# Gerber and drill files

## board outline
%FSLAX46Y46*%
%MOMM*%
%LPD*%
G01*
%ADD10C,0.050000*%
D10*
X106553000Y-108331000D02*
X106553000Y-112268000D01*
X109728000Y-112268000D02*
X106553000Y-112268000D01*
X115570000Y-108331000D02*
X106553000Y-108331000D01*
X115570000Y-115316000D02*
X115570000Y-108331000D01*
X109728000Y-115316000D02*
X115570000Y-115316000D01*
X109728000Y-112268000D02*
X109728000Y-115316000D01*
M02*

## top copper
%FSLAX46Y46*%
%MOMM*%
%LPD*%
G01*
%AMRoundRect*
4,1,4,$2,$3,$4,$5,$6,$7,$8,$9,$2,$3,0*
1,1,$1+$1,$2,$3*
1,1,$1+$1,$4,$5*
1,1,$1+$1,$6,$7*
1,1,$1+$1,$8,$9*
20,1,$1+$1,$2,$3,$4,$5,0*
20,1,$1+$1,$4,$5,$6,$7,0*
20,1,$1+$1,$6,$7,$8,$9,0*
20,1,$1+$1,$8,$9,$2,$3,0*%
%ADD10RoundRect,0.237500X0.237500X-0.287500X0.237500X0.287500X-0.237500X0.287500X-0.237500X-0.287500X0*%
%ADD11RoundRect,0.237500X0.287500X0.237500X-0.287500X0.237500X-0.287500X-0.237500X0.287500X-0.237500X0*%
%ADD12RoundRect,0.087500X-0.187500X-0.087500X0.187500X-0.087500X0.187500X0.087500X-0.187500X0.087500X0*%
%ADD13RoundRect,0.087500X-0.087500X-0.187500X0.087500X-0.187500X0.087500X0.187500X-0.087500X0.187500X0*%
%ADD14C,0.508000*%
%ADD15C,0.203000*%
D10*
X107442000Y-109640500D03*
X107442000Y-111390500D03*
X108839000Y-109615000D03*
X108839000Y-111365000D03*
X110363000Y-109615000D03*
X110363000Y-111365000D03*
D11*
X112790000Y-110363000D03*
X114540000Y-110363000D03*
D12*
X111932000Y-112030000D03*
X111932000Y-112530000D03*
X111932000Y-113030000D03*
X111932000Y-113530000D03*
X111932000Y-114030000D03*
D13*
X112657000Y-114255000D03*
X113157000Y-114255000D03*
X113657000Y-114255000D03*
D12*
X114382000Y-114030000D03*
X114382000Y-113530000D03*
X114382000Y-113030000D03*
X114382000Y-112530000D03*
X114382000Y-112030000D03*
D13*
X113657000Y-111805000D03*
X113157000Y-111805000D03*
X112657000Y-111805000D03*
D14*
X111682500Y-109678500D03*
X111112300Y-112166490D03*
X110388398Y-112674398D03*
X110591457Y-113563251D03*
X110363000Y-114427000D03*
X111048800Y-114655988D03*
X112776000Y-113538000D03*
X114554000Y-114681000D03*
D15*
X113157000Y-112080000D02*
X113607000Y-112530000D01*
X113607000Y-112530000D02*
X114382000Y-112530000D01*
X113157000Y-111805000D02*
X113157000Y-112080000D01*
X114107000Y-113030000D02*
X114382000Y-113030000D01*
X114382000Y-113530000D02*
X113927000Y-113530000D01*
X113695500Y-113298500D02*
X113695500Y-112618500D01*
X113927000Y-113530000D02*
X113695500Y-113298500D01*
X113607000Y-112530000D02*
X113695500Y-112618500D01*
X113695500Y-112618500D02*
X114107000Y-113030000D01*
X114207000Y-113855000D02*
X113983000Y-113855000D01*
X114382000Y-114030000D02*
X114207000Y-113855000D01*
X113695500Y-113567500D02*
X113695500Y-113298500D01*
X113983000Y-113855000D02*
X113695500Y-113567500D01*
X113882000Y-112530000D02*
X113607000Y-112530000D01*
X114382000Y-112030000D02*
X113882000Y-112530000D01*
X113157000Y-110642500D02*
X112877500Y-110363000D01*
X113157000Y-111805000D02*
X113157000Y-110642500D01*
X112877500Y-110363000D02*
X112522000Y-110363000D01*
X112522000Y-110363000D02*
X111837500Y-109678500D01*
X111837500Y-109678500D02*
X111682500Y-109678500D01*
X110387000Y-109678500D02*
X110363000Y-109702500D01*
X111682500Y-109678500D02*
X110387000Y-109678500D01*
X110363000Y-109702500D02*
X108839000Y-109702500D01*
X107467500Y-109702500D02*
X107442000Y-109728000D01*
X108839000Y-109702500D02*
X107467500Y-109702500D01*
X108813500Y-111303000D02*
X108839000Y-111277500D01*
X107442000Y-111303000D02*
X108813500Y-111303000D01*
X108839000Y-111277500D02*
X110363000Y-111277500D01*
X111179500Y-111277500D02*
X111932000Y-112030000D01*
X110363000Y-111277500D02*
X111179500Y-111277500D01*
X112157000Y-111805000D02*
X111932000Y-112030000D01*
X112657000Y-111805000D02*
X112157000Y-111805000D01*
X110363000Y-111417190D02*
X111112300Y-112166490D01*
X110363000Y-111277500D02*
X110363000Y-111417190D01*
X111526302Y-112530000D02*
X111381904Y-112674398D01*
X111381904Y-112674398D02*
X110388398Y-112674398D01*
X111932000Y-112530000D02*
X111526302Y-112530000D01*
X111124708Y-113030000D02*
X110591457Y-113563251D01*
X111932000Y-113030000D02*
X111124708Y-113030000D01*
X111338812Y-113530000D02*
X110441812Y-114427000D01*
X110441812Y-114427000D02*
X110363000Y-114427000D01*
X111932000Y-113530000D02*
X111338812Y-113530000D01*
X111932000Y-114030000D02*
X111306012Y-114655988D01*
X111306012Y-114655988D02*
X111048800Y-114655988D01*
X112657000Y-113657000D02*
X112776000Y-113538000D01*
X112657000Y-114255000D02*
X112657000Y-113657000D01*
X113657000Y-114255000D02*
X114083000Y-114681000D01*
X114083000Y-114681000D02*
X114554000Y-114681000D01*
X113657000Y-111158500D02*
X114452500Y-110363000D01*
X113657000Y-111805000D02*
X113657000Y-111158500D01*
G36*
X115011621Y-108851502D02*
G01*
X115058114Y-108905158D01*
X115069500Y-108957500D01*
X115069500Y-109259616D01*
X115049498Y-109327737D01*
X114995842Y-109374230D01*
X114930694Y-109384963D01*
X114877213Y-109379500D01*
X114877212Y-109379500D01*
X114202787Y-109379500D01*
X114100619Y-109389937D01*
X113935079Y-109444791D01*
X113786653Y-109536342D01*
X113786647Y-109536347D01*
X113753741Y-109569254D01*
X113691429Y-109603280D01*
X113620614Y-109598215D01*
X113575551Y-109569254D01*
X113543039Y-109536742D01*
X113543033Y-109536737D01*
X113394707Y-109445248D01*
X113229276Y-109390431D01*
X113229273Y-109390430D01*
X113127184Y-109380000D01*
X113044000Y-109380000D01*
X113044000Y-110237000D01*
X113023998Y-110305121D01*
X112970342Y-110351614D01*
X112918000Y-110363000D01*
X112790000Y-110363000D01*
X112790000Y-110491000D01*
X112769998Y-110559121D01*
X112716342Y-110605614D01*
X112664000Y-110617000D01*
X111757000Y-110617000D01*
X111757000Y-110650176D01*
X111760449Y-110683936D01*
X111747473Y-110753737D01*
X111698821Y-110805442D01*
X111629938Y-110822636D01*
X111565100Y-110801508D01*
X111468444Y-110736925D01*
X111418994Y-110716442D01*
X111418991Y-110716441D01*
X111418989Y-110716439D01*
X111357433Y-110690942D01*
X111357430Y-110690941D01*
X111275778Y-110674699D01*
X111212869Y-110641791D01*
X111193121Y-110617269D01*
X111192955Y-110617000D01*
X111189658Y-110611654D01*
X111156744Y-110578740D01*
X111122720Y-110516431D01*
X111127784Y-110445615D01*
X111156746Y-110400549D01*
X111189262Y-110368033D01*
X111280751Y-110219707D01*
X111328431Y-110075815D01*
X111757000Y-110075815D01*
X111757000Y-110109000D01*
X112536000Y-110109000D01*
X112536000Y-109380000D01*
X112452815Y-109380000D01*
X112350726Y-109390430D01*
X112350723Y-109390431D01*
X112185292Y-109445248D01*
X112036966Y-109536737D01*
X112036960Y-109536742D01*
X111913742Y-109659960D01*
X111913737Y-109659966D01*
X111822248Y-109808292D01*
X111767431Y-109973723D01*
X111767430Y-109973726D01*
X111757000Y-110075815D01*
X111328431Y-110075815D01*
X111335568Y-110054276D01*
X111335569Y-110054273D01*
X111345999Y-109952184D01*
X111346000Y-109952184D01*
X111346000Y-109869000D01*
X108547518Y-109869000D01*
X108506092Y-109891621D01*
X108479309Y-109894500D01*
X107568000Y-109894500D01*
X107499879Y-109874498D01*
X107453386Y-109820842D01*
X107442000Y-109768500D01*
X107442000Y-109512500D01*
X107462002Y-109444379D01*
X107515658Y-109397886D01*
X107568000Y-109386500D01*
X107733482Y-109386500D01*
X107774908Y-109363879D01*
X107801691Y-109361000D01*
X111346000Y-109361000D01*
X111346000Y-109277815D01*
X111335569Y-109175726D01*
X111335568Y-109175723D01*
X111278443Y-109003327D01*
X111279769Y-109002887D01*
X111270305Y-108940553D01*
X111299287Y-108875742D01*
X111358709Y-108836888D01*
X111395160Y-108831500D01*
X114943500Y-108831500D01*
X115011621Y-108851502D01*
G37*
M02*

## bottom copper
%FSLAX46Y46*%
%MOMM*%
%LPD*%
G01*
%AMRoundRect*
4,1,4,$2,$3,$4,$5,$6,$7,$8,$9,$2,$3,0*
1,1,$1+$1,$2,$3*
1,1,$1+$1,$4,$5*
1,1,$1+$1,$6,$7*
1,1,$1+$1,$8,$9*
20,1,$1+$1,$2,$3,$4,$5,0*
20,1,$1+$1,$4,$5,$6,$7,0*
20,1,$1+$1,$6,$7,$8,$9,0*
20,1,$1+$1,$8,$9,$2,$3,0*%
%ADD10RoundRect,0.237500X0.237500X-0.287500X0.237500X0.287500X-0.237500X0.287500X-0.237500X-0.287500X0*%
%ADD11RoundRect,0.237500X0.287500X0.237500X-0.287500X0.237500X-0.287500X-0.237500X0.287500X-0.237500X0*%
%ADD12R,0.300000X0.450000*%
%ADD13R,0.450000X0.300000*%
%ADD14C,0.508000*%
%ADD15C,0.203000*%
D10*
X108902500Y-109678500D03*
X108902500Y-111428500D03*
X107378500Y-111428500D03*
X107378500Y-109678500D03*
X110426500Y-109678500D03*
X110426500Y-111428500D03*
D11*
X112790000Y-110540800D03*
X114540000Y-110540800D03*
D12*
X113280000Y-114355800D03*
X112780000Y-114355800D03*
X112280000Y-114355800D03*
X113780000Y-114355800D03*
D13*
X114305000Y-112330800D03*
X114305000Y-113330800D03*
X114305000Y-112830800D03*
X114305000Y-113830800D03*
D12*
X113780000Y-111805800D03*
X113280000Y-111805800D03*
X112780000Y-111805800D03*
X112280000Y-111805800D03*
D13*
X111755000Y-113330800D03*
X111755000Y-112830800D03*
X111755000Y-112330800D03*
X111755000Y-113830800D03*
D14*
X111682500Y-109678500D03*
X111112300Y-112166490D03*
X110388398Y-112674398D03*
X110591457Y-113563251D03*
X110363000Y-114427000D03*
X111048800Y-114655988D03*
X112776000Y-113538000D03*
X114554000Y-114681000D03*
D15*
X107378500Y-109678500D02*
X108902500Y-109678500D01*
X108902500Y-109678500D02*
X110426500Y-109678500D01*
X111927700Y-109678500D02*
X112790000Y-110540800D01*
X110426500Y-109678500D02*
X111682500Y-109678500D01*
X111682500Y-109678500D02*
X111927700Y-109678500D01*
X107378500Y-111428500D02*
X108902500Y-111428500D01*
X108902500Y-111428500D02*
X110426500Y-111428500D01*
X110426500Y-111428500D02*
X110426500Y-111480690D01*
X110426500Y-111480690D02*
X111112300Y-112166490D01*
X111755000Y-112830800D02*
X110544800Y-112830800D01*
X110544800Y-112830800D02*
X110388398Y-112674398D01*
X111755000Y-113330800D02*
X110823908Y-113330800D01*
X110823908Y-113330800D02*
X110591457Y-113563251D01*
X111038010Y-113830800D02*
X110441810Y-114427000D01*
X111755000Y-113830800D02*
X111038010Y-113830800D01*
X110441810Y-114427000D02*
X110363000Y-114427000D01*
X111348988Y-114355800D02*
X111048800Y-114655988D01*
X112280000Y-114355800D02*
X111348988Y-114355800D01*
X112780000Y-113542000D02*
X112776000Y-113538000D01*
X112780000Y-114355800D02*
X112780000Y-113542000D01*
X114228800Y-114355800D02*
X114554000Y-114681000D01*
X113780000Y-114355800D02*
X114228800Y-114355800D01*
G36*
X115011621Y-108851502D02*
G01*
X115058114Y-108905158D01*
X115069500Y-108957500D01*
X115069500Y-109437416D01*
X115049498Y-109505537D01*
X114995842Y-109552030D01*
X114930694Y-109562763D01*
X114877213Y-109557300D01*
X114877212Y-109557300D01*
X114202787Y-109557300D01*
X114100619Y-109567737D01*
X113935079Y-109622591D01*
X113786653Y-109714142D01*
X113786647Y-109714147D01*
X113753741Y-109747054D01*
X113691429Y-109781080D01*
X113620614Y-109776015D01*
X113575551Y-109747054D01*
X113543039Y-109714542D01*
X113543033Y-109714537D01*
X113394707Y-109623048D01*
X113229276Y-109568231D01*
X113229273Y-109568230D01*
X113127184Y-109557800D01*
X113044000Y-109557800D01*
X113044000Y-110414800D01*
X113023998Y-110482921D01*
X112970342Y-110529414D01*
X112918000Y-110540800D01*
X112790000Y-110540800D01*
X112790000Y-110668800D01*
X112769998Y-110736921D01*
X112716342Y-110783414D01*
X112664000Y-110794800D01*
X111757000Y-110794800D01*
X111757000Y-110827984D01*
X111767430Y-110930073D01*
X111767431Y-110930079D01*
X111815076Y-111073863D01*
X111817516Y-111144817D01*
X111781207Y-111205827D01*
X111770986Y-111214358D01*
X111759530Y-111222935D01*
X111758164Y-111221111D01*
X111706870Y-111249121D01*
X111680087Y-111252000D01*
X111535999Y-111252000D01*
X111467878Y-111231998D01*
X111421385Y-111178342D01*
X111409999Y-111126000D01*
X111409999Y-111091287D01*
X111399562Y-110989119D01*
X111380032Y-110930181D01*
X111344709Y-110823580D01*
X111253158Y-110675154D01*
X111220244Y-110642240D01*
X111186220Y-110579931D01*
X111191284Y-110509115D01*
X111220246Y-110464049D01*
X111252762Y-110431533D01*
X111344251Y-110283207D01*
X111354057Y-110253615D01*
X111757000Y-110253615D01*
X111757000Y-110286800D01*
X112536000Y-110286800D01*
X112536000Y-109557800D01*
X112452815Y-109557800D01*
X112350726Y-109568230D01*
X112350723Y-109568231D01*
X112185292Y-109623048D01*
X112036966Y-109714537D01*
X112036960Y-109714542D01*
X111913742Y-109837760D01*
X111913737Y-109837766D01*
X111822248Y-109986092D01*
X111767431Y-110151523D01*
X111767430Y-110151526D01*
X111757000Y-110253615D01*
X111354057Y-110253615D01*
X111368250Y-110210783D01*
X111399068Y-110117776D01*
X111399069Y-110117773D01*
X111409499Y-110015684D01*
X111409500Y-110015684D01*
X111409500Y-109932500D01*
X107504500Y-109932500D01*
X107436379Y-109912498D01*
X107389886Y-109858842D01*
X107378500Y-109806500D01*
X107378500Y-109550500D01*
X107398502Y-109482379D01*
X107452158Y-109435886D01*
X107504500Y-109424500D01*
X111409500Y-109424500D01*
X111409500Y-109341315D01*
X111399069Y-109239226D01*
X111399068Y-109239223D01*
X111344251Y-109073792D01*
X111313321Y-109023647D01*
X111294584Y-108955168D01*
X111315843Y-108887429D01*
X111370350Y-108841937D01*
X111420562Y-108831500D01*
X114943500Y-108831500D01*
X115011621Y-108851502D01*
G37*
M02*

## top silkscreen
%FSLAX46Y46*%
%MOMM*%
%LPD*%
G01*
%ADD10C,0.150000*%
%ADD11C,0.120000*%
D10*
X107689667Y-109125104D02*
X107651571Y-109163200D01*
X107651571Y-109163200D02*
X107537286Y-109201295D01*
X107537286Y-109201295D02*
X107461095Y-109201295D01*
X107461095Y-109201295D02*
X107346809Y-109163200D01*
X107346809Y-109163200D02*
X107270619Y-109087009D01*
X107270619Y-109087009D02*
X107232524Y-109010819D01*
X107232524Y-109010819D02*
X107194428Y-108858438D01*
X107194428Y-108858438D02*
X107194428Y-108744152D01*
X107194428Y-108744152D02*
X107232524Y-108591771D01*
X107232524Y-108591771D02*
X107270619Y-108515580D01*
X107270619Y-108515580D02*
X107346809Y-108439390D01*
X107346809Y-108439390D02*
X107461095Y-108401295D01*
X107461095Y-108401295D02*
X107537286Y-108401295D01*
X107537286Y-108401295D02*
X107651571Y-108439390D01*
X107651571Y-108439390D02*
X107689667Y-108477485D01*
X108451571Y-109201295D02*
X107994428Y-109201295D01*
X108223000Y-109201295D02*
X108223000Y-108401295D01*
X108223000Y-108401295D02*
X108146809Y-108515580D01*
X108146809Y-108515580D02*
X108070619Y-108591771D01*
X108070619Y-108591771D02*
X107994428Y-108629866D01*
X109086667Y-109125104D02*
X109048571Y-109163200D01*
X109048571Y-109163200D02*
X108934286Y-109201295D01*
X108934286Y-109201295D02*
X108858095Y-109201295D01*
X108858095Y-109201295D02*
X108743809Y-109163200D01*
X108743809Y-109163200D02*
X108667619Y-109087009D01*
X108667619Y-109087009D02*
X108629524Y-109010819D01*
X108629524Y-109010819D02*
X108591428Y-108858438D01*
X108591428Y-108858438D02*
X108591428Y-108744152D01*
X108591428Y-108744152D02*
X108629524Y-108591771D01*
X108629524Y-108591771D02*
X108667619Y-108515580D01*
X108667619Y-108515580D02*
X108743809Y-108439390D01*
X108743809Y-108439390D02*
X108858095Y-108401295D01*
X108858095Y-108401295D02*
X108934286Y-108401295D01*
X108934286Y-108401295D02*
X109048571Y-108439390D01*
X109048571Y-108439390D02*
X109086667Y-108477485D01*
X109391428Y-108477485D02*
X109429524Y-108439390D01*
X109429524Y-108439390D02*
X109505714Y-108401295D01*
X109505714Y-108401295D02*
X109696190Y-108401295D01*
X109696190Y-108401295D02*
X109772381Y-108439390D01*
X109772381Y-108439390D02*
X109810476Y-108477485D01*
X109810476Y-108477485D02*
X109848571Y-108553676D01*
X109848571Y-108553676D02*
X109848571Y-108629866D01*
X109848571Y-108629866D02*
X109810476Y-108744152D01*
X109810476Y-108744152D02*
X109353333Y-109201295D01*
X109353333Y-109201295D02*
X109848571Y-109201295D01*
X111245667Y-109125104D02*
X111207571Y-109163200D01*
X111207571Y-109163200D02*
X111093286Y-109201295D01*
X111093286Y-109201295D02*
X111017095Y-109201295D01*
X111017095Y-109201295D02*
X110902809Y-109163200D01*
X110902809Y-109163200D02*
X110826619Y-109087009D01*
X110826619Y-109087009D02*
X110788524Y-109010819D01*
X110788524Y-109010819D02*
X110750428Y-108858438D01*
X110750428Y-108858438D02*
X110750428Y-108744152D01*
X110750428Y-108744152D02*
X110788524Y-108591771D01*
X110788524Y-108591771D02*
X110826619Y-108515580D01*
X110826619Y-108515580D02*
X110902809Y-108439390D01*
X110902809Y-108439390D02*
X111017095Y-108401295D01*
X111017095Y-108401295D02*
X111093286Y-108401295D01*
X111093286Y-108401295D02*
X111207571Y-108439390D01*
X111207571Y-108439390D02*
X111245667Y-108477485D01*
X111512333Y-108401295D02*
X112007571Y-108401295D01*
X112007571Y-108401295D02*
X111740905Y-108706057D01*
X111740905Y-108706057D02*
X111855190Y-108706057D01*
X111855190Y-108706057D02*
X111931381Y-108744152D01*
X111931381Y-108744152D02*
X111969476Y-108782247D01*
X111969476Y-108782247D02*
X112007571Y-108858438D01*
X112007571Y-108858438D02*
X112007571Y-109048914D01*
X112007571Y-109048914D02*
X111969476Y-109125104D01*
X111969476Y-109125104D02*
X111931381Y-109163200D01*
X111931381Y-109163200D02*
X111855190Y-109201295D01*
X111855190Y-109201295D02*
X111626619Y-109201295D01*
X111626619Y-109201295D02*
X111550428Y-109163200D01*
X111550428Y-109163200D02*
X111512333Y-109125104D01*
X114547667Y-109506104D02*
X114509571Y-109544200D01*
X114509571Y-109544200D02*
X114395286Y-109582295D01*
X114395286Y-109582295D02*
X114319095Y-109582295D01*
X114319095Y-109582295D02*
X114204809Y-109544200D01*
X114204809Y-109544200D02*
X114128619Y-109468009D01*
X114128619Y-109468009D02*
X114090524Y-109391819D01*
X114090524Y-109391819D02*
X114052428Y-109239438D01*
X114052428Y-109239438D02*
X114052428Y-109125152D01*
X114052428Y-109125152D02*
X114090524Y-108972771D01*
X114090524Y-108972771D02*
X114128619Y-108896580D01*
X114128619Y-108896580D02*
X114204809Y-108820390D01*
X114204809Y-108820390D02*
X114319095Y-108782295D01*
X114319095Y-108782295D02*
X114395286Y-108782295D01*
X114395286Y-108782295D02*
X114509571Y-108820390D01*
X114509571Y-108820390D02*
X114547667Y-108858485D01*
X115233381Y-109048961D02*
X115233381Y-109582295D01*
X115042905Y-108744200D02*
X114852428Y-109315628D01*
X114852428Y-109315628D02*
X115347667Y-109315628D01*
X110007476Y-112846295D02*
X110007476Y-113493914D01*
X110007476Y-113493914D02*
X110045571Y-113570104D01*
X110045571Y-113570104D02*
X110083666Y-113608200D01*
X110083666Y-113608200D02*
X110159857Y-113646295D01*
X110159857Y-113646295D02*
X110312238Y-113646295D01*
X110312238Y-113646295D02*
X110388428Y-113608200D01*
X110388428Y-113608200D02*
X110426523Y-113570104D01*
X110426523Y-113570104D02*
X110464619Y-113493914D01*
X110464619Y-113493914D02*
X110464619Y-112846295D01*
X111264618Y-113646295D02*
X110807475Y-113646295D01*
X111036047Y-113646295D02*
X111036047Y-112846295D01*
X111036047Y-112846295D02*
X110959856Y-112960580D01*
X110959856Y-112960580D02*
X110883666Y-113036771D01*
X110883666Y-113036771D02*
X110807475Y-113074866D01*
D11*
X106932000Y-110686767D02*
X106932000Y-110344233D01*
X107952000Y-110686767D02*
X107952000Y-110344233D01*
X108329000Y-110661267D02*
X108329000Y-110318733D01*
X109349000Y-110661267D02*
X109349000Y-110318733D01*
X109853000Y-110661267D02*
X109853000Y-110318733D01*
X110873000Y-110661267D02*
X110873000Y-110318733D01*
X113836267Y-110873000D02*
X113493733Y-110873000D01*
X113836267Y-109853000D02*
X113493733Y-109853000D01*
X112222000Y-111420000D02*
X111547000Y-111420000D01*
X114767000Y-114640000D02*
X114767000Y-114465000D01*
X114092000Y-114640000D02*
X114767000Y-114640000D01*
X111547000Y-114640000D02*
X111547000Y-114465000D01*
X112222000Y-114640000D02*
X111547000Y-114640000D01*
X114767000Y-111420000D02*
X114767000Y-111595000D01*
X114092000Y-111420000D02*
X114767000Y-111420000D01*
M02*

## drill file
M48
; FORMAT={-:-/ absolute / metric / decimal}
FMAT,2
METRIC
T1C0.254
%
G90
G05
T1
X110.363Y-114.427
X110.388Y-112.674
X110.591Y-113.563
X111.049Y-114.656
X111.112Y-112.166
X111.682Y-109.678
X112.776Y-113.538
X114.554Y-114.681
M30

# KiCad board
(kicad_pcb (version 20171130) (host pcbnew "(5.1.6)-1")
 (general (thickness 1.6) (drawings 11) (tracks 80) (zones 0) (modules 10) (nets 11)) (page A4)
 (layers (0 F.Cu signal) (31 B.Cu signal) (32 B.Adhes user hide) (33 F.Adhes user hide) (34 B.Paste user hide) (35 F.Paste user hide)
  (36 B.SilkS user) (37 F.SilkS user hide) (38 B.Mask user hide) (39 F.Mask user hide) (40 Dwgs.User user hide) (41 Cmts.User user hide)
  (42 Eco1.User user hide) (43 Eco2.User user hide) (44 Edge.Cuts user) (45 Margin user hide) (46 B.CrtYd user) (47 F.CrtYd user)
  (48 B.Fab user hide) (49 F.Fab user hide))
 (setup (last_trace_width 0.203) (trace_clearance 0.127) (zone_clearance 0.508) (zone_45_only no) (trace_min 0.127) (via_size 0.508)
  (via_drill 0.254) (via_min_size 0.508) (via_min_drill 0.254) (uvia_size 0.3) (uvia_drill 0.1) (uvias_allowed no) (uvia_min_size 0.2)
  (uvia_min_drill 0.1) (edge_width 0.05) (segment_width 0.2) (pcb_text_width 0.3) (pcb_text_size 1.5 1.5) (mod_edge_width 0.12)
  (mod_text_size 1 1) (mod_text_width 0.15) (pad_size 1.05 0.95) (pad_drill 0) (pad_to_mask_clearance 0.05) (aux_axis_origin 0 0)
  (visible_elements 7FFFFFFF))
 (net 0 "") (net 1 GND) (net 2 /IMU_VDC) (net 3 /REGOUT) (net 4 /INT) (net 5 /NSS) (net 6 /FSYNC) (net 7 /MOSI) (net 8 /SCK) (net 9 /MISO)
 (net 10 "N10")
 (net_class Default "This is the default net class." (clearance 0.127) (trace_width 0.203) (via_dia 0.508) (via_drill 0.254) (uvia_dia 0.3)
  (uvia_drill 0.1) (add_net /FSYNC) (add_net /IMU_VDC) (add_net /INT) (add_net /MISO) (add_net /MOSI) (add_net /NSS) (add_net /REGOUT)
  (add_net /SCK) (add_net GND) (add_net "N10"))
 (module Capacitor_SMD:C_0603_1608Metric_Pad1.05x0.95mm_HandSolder (layer F.Cu) (at 107.442 110.5155 90)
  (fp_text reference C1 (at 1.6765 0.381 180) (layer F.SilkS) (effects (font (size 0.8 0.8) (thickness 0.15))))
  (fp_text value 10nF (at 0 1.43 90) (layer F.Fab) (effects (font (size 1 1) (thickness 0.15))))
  (fp_line (start -0.171267 -0.51) (end 0.171267 -0.51) (layer F.SilkS) (width 0.12))
  (fp_line (start -0.171267 0.51) (end 0.171267 0.51) (layer F.SilkS) (width 0.12))
  (pad 2 smd roundrect (at 0.875 0 90) (size 1.05 0.95) (layers F.Cu F.Paste F.Mask) (roundrect_rratio 0.25) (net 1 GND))
  (pad 1 smd roundrect (at -0.875 0 90) (size 1.05 0.95) (layers F.Cu F.Paste F.Mask) (roundrect_rratio 0.25) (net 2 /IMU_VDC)))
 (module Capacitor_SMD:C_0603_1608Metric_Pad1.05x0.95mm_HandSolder (layer F.Cu) (at 108.839 110.49 90)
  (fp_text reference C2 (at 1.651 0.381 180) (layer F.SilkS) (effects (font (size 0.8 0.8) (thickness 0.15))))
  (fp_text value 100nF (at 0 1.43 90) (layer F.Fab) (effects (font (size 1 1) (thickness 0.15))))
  (fp_line (start -0.171267 -0.51) (end 0.171267 -0.51) (layer F.SilkS) (width 0.12))
  (fp_line (start -0.171267 0.51) (end 0.171267 0.51) (layer F.SilkS) (width 0.12))
  (pad 2 smd roundrect (at 0.875 0 90) (size 1.05 0.95) (layers F.Cu F.Paste F.Mask) (roundrect_rratio 0.25) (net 1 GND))
  (pad 1 smd roundrect (at -0.875 0 90) (size 1.05 0.95) (layers F.Cu F.Paste F.Mask) (roundrect_rratio 0.25) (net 2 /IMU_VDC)))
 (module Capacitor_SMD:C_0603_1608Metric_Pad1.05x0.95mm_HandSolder (layer F.Cu) (at 110.363 110.49 90)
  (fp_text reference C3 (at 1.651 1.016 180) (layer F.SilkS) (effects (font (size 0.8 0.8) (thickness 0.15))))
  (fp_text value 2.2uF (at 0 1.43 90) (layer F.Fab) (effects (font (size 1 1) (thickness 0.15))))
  (fp_line (start -0.171267 -0.51) (end 0.171267 -0.51) (layer F.SilkS) (width 0.12))
  (fp_line (start -0.171267 0.51) (end 0.171267 0.51) (layer F.SilkS) (width 0.12))
  (pad 2 smd roundrect (at 0.875 0 90) (size 1.05 0.95) (layers F.Cu F.Paste F.Mask) (roundrect_rratio 0.25) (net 1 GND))
  (pad 1 smd roundrect (at -0.875 0 90) (size 1.05 0.95) (layers F.Cu F.Paste F.Mask) (roundrect_rratio 0.25) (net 2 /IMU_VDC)))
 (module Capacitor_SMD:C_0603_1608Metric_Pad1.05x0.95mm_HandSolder (layer F.Cu) (at 113.665 110.363 180)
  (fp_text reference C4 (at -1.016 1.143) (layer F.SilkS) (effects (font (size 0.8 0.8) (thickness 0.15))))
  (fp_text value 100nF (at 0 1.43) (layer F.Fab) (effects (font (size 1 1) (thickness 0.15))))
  (fp_line (start -0.171267 -0.51) (end 0.171267 -0.51) (layer F.SilkS) (width 0.12))
  (fp_line (start -0.171267 0.51) (end 0.171267 0.51) (layer F.SilkS) (width 0.12))
  (pad 2 smd roundrect (at 0.875 0 180) (size 1.05 0.95) (layers F.Cu F.Paste F.Mask) (roundrect_rratio 0.25) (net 1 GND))
  (pad 1 smd roundrect (at -0.875 0 180) (size 1.05 0.95) (layers F.Cu F.Paste F.Mask) (roundrect_rratio 0.25) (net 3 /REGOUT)))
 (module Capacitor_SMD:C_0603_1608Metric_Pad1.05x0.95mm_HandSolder (layer B.Cu) (at 108.9025 110.5535 90)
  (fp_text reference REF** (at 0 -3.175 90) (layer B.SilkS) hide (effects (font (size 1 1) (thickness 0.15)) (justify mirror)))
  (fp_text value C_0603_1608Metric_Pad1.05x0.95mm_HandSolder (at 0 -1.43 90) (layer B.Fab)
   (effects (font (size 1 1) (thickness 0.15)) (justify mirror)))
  (pad 2 smd roundrect (at 0.875 0 90) (size 1.05 0.95) (layers B.Cu B.Paste B.Mask) (roundrect_rratio 0.25) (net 1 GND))
  (pad 1 smd roundrect (at -0.875 0 90) (size 1.05 0.95) (layers B.Cu B.Paste B.Mask) (roundrect_rratio 0.25) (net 2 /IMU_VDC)))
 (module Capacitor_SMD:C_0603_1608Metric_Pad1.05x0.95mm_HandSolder (layer B.Cu) (at 107.3785 110.5535 90)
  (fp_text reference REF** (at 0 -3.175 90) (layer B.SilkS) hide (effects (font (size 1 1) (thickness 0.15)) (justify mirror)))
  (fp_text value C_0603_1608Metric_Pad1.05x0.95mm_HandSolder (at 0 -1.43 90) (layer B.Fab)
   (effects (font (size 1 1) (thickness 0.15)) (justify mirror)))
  (pad 1 smd roundrect (at -0.875 0 90) (size 1.05 0.95) (layers B.Cu B.Paste B.Mask) (roundrect_rratio 0.25) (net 2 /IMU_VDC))
  (pad 2 smd roundrect (at 0.875 0 90) (size 1.05 0.95) (layers B.Cu B.Paste B.Mask) (roundrect_rratio 0.25) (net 1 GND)))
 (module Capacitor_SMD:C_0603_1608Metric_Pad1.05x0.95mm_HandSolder (layer B.Cu) (at 110.4265 110.5535 90)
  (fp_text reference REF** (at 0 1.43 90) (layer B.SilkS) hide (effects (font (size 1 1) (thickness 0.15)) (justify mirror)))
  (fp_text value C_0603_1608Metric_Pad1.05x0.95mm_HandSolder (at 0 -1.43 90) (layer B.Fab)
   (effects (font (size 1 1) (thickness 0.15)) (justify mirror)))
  (pad 2 smd roundrect (at 0.875 0 90) (size 1.05 0.95) (layers B.Cu B.Paste B.Mask) (roundrect_rratio 0.25) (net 1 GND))
  (pad 1 smd roundrect (at -0.875 0 90) (size 1.05 0.95) (layers B.Cu B.Paste B.Mask) (roundrect_rratio 0.25) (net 2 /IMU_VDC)))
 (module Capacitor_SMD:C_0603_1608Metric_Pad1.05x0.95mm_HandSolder (layer B.Cu) (at 113.665 110.5408 180)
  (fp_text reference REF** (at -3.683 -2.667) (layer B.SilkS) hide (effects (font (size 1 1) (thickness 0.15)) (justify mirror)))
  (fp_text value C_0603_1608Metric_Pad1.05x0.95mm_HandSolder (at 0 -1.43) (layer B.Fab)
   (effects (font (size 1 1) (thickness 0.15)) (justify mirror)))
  (pad 2 smd roundrect (at 0.875 0 180) (size 1.05 0.95) (layers B.Cu B.Paste B.Mask) (roundrect_rratio 0.25) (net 1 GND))
  (pad 1 smd roundrect (at -0.875 0 180) (size 1.05 0.95) (layers B.Cu B.Paste B.Mask) (roundrect_rratio 0.25)))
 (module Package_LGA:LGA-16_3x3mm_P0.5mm (layer B.Cu) (at 113.03 113.0808 270)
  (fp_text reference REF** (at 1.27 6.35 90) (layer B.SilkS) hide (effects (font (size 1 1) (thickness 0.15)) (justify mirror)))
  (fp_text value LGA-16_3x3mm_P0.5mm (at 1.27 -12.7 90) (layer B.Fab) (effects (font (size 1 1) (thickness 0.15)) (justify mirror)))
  (pad 10 smd rect (at 1.275 -0.25 180) (size 0.3 0.45) (layers B.Cu B.Paste B.Mask))
  (pad 11 smd rect (at 1.275 0.25 180) (size 0.3 0.45) (layers B.Cu B.Paste B.Mask) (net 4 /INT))
  (pad 12 smd rect (at 1.275 0.75 180) (size 0.3 0.45) (layers B.Cu B.Paste B.Mask) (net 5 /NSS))
  (pad 9 smd rect (at 1.275 -0.75 180) (size 0.3 0.45) (layers B.Cu B.Paste B.Mask) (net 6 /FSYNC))
  (pad 5 smd rect (at -0.75 -1.275 270) (size 0.3 0.45) (layers B.Cu B.Paste B.Mask))
  (pad 7 smd rect (at 0.25 -1.275 270) (size 0.3 0.45) (layers B.Cu B.Paste B.Mask))
  (pad 6 smd rect (at -0.25 -1.275 270) (size 0.3 0.45) (layers B.Cu B.Paste B.Mask))
  (pad 8 smd rect (at 0.75 -1.275 270) (size 0.3 0.45) (layers B.Cu B.Paste B.Mask))
  (pad 4 smd rect (at -1.275 -0.75 180) (size 0.3 0.45) (layers B.Cu B.Paste B.Mask))
  (pad 3 smd rect (at -1.275 -0.25 180) (size 0.3 0.45) (layers B.Cu B.Paste B.Mask))
  (pad 2 smd rect (at -1.275 0.25 180) (size 0.3 0.45) (layers B.Cu B.Paste B.Mask))
  (pad 1 smd rect (at -1.275 0.75 180) (size 0.3 0.45) (layers B.Cu B.Paste B.Mask))
  (pad 14 smd rect (at 0.25 1.275 270) (size 0.3 0.45) (layers B.Cu B.Paste B.Mask) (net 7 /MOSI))
  (pad 15 smd rect (at -0.25 1.275 270) (size 0.3 0.45) (layers B.Cu B.Paste B.Mask) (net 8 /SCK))
  (pad 16 smd rect (at -0.75 1.275 270) (size 0.3 0.45) (layers B.Cu B.Paste B.Mask))
  (pad 13 smd rect (at 0.75 1.275 270) (size 0.3 0.45) (layers B.Cu B.Paste B.Mask) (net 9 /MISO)))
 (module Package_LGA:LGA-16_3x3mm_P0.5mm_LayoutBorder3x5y (layer F.Cu) (at 113.157 113.03)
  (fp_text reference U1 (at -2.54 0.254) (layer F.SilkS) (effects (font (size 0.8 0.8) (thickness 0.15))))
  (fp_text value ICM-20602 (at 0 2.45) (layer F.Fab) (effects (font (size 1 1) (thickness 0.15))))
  (fp_line (start -0.935 -1.61) (end -1.61 -1.61) (layer F.SilkS) (width 0.12))
  (fp_line (start 1.61 1.61) (end 1.61 1.435) (layer F.SilkS) (width 0.12))
  (fp_line (start 0.935 1.61) (end 1.61 1.61) (layer F.SilkS) (width 0.12))
  (fp_line (start -1.61 1.61) (end -1.61 1.435) (layer F.SilkS) (width 0.12))
  (fp_line (start -0.935 1.61) (end -1.61 1.61) (layer F.SilkS) (width 0.12))
  (fp_line (start 1.61 -1.61) (end 1.61 -1.435) (layer F.SilkS) (width 0.12))
  (fp_line (start 0.935 -1.61) (end 1.61 -1.61) (layer F.SilkS) (width 0.12))
  (pad 1 smd roundrect (at -1.225 -1) (size 0.55 0.35) (layers F.Cu F.Paste F.Mask) (roundrect_rratio 0.25) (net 2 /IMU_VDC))
  (pad 2 smd roundrect (at -1.225 -0.5) (size 0.55 0.35) (layers F.Cu F.Paste F.Mask) (roundrect_rratio 0.25) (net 8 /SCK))
  (pad 3 smd roundrect (at -1.225 0) (size 0.55 0.35) (layers F.Cu F.Paste F.Mask) (roundrect_rratio 0.25) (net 7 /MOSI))
  (pad 4 smd roundrect (at -1.225 0.5) (size 0.55 0.35) (layers F.Cu F.Paste F.Mask) (roundrect_rratio 0.25) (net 9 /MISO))
  (pad 5 smd roundrect (at -1.225 1) (size 0.55 0.35) (layers F.Cu F.Paste F.Mask) (roundrect_rratio 0.25) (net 5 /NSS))
  (pad 6 smd roundrect (at -0.5 1.225) (size 0.35 0.55) (layers F.Cu F.Paste F.Mask) (roundrect_rratio 0.25) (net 4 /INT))
  (pad 7 smd roundrect (at 0 1.225) (size 0.35 0.55) (layers F.Cu F.Paste F.Mask) (roundrect_rratio 0.25) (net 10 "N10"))
  (pad 8 smd roundrect (at 0.5 1.225) (size 0.35 0.55) (layers F.Cu F.Paste F.Mask) (roundrect_rratio 0.25) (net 6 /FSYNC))
  (pad 9 smd roundrect (at 1.225 1) (size 0.55 0.35) (layers F.Cu F.Paste F.Mask) (roundrect_rratio 0.25) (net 1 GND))
  (pad 10 smd roundrect (at 1.225 0.5) (size 0.55 0.35) (layers F.Cu F.Paste F.Mask) (roundrect_rratio 0.25) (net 1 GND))
  (pad 11 smd roundrect (at 1.225 0) (size 0.55 0.35) (layers F.Cu F.Paste F.Mask) (roundrect_rratio 0.25) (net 1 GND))
  (pad 12 smd roundrect (at 1.225 -0.5) (size 0.55 0.35) (layers F.Cu F.Paste F.Mask) (roundrect_rratio 0.25) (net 1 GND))
  (pad 13 smd roundrect (at 1.225 -1) (size 0.55 0.35) (layers F.Cu F.Paste F.Mask) (roundrect_rratio 0.25) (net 1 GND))
  (pad 14 smd roundrect (at 0.5 -1.225) (size 0.35 0.55) (layers F.Cu F.Paste F.Mask) (roundrect_rratio 0.25) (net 3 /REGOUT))
  (pad 15 smd roundrect (at 0 -1.225) (size 0.35 0.55) (layers F.Cu F.Paste F.Mask) (roundrect_rratio 0.25) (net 1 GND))
  (pad 16 smd roundrect (at -0.5 -1.225) (size 0.35 0.55) (layers F.Cu F.Paste F.Mask) (roundrect_rratio 0.25) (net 2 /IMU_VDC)))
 (gr_line (start 106.553 108.331) (end 106.553 112.268) (layer Edge.Cuts) (width 0.05))
 (gr_line (start 109.728 112.268) (end 106.553 112.268) (layer Edge.Cuts) (width 0.05))
 (gr_line (start 115.57 108.331) (end 106.553 108.331) (layer Edge.Cuts) (width 0.05))
 (gr_line (start 115.57 115.316) (end 115.57 108.331) (layer Edge.Cuts) (width 0.05))
 (gr_line (start 109.728 115.316) (end 115.57 115.316) (layer Edge.Cuts) (width 0.05))
 (gr_line (start 109.728 112.268) (end 109.728 115.316) (layer Edge.Cuts) (width 0.05))
 (segment (start 107.3785 109.6785) (end 108.9025 109.6785) (width 0.203) (layer B.Cu) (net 1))
 (segment (start 108.9025 109.6785) (end 110.4265 109.6785) (width 0.203) (layer B.Cu) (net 1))
 (segment (start 111.9277 109.6785) (end 112.79 110.5408) (width 0.203) (layer B.Cu) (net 1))
 (segment (start 113.157 112.08) (end 113.607 112.53) (width 0.203) (layer F.Cu) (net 1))
 (segment (start 113.607 112.53) (end 114.382 112.53) (width 0.203) (layer F.Cu) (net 1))
 (segment (start 113.157 111.805) (end 113.157 112.08) (width 0.203) (layer F.Cu) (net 1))
 (segment (start 114.107 113.03) (end 114.382 113.03) (width 0.203) (layer F.Cu) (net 1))
 (segment (start 114.382 113.53) (end 113.927 113.53) (width 0.203) (layer F.Cu) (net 1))
 (segment (start 113.6955 113.2985) (end 113.6955 112.6185) (width 0.203) (layer F.Cu) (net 1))
 (segment (start 113.927 113.53) (end 113.6955 113.2985) (width 0.203) (layer F.Cu) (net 1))
 (segment (start 113.607 112.53) (end 113.6955 112.6185) (width 0.203) (layer F.Cu) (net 1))
 (segment (start 113.6955 112.6185) (end 114.107 113.03) (width 0.203) (layer F.Cu) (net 1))
 (segment (start 114.207 113.855) (end 113.983 113.855) (width 0.203) (layer F.Cu) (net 1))
 (segment (start 114.382 114.03) (end 114.207 113.855) (width 0.203) (layer F.Cu) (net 1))
 (segment (start 113.6955 113.5675) (end 113.6955 113.2985) (width 0.203) (layer F.Cu) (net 1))
 (segment (start 113.983 113.855) (end 113.6955 113.5675) (width 0.203) (layer F.Cu) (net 1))
 (segment (start 113.882 112.53) (end 113.607 112.53) (width 0.203) (layer F.Cu) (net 1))
 (segment (start 114.382 112.03) (end 113.882 112.53) (width 0.203) (layer F.Cu) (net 1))
 (segment (start 113.157 110.6425) (end 112.8775 110.363) (width 0.203) (layer F.Cu) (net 1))
 (segment (start 113.157 111.805) (end 113.157 110.6425) (width 0.203) (layer F.Cu) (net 1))
 (segment (start 112.8775 110.363) (end 112.522 110.363) (width 0.203) (layer F.Cu) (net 1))
 (via (at 111.6825 109.6785) (size 0.508) (drill 0.254) (layers F.Cu B.Cu) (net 1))
 (segment (start 112.522 110.363) (end 111.8375 109.6785) (width 0.203) (layer F.Cu) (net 1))
 (segment (start 111.8375 109.6785) (end 111.6825 109.6785) (width 0.203) (layer F.Cu) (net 1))
 (segment (start 110.4265 109.6785) (end 111.6825 109.6785) (width 0.203) (layer B.Cu) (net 1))
 (segment (start 111.6825 109.6785) (end 111.9277 109.6785) (width 0.203) (layer B.Cu) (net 1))
 (segment (start 110.387 109.6785) (end 110.363 109.7025) (width 0.203) (layer F.Cu) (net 1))
 (segment (start 111.6825 109.6785) (end 110.387 109.6785) (width 0.203) (layer F.Cu) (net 1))
 (segment (start 110.363 109.7025) (end 108.839 109.7025) (width 0.203) (layer F.Cu) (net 1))
 (segment (start 107.4675 109.7025) (end 107.442 109.728) (width 0.203) (layer F.Cu) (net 1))
 (segment (start 108.839 109.7025) (end 107.4675 109.7025) (width 0.203) (layer F.Cu) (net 1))
 (segment (start 107.3785 111.4285) (end 108.9025 111.4285) (width 0.203) (layer B.Cu) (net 2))
 (segment (start 108.9025 111.4285) (end 110.4265 111.4285) (width 0.203) (layer B.Cu) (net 2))
 (segment (start 108.8135 111.303) (end 108.839 111.2775) (width 0.203) (layer F.Cu) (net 2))
 (segment (start 107.442 111.303) (end 108.8135 111.303) (width 0.203) (layer F.Cu) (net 2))
 (segment (start 108.839 111.2775) (end 110.363 111.2775) (width 0.203) (layer F.Cu) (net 2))
 (segment (start 111.1795 111.2775) (end 111.932 112.03) (width 0.203) (layer F.Cu) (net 2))
 (segment (start 110.363 111.2775) (end 111.1795 111.2775) (width 0.203) (layer F.Cu) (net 2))
 (segment (start 112.157 111.805) (end 111.932 112.03) (width 0.203) (layer F.Cu) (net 2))
 (segment (start 112.657 111.805) (end 112.157 111.805) (width 0.203) (layer F.Cu) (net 2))
 (segment (start 110.363 111.41719) (end 111.1123 112.16649) (width 0.203) (layer F.Cu) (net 2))
 (via (at 111.1123 112.16649) (size 0.508) (drill 0.254) (layers F.Cu B.Cu) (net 2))
 (segment (start 110.4265 111.4285) (end 110.4265 111.48069) (width 0.203) (layer B.Cu) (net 2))
 (segment (start 110.4265 111.48069) (end 111.1123 112.16649) (width 0.203) (layer B.Cu) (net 2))
 (segment (start 110.363 111.2775) (end 110.363 111.41719) (width 0.203) (layer F.Cu) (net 2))
 (segment (start 111.755 112.8308) (end 110.5448 112.8308) (width 0.203) (layer B.Cu) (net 8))
 (segment (start 111.526302 112.53) (end 111.381904 112.674398) (width 0.203) (layer F.Cu) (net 8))
 (via (at 110.388398 112.674398) (size 0.508) (drill 0.254) (layers F.Cu B.Cu) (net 8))
 (segment (start 111.381904 112.674398) (end 110.388398 112.674398) (width 0.203) (layer F.Cu) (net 8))
 (segment (start 111.932 112.53) (end 111.526302 112.53) (width 0.203) (layer F.Cu) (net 8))
 (segment (start 110.5448 112.8308) (end 110.388398 112.674398) (width 0.203) (layer B.Cu) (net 8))
 (segment (start 111.124708 113.03) (end 110.591457 113.563251) (width 0.203) (layer F.Cu) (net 7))
 (segment (start 111.755 113.3308) (end 110.823908 113.3308) (width 0.203) (layer B.Cu) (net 7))
 (via (at 110.591457 113.563251) (size 0.508) (drill 0.254) (layers F.Cu B.Cu) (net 7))
 (segment (start 110.823908 113.3308) (end 110.591457 113.563251) (width 0.203) (layer B.Cu) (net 7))
 (segment (start 111.932 113.03) (end 111.124708 113.03) (width 0.203) (layer F.Cu) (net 7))
 (segment (start 111.338812 113.53) (end 110.441812 114.427) (width 0.203) (layer F.Cu) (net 9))
 (segment (start 111.03801 113.8308) (end 110.44181 114.427) (width 0.203) (layer B.Cu) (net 9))
 (segment (start 110.441812 114.427) (end 110.363 114.427) (width 0.203) (layer F.Cu) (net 9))
 (via (at 110.363 114.427) (size 0.508) (drill 0.254) (layers F.Cu B.Cu) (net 9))
 (segment (start 111.755 113.8308) (end 111.03801 113.8308) (width 0.203) (layer B.Cu) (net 9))
 (segment (start 111.932 113.53) (end 111.338812 113.53) (width 0.203) (layer F.Cu) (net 9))
 (segment (start 110.44181 114.427) (end 110.363 114.427) (width 0.203) (layer B.Cu) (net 9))
 (via (at 111.0488 114.655988) (size 0.508) (drill 0.254) (layers F.Cu B.Cu) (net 5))
 (segment (start 111.932 114.03) (end 111.306012 114.655988) (width 0.203) (layer F.Cu) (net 5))
 (segment (start 111.348988 114.3558) (end 111.0488 114.655988) (width 0.203) (layer B.Cu) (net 5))
 (segment (start 111.306012 114.655988) (end 111.0488 114.655988) (width 0.203) (layer F.Cu) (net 5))
 (segment (start 112.28 114.3558) (end 111.348988 114.3558) (width 0.203) (layer B.Cu) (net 5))
 (via (at 112.776 113.538) (size 0.508) (drill 0.254) (layers F.Cu B.Cu) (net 4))
 (segment (start 112.78 113.542) (end 112.776 113.538) (width 0.203) (layer B.Cu) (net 4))
 (segment (start 112.78 114.3558) (end 112.78 113.542) (width 0.203) (layer B.Cu) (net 4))
 (segment (start 112.657 113.657) (end 112.776 113.538) (width 0.203) (layer F.Cu) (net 4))
 (segment (start 112.657 114.255) (end 112.657 113.657) (width 0.203) (layer F.Cu) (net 4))
 (segment (start 114.2288 114.3558) (end 114.554 114.681) (width 0.203) (layer B.Cu) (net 6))
 (segment (start 113.78 114.3558) (end 114.2288 114.3558) (width 0.203) (layer B.Cu) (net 6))
 (segment (start 113.657 114.255) (end 114.083 114.681) (width 0.203) (layer F.Cu) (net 6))
 (segment (start 114.083 114.681) (end 114.554 114.681) (width 0.203) (layer F.Cu) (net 6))
 (via (at 114.554 114.681) (size 0.508) (drill 0.254) (layers F.Cu B.Cu) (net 6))
 (segment (start 113.657 111.1585) (end 114.4525 110.363) (width 0.203) (layer F.Cu) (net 3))
 (segment (start 113.657 111.805) (end 113.657 111.1585) (width 0.203) (layer F.Cu) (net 3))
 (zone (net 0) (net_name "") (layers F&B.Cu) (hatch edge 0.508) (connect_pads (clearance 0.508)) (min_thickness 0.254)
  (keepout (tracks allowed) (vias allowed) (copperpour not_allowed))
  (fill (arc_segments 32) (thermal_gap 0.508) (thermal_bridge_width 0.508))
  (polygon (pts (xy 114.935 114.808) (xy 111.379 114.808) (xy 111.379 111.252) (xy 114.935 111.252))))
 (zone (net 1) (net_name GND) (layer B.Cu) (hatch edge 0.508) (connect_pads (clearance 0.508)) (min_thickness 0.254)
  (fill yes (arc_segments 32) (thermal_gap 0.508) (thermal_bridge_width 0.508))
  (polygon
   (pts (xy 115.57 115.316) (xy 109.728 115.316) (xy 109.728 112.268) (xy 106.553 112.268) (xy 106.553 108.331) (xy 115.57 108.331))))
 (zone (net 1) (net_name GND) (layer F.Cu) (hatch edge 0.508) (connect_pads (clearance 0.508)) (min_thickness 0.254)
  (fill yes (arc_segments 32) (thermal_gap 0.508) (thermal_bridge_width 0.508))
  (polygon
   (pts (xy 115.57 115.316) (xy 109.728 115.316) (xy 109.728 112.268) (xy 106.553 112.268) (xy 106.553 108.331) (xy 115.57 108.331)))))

